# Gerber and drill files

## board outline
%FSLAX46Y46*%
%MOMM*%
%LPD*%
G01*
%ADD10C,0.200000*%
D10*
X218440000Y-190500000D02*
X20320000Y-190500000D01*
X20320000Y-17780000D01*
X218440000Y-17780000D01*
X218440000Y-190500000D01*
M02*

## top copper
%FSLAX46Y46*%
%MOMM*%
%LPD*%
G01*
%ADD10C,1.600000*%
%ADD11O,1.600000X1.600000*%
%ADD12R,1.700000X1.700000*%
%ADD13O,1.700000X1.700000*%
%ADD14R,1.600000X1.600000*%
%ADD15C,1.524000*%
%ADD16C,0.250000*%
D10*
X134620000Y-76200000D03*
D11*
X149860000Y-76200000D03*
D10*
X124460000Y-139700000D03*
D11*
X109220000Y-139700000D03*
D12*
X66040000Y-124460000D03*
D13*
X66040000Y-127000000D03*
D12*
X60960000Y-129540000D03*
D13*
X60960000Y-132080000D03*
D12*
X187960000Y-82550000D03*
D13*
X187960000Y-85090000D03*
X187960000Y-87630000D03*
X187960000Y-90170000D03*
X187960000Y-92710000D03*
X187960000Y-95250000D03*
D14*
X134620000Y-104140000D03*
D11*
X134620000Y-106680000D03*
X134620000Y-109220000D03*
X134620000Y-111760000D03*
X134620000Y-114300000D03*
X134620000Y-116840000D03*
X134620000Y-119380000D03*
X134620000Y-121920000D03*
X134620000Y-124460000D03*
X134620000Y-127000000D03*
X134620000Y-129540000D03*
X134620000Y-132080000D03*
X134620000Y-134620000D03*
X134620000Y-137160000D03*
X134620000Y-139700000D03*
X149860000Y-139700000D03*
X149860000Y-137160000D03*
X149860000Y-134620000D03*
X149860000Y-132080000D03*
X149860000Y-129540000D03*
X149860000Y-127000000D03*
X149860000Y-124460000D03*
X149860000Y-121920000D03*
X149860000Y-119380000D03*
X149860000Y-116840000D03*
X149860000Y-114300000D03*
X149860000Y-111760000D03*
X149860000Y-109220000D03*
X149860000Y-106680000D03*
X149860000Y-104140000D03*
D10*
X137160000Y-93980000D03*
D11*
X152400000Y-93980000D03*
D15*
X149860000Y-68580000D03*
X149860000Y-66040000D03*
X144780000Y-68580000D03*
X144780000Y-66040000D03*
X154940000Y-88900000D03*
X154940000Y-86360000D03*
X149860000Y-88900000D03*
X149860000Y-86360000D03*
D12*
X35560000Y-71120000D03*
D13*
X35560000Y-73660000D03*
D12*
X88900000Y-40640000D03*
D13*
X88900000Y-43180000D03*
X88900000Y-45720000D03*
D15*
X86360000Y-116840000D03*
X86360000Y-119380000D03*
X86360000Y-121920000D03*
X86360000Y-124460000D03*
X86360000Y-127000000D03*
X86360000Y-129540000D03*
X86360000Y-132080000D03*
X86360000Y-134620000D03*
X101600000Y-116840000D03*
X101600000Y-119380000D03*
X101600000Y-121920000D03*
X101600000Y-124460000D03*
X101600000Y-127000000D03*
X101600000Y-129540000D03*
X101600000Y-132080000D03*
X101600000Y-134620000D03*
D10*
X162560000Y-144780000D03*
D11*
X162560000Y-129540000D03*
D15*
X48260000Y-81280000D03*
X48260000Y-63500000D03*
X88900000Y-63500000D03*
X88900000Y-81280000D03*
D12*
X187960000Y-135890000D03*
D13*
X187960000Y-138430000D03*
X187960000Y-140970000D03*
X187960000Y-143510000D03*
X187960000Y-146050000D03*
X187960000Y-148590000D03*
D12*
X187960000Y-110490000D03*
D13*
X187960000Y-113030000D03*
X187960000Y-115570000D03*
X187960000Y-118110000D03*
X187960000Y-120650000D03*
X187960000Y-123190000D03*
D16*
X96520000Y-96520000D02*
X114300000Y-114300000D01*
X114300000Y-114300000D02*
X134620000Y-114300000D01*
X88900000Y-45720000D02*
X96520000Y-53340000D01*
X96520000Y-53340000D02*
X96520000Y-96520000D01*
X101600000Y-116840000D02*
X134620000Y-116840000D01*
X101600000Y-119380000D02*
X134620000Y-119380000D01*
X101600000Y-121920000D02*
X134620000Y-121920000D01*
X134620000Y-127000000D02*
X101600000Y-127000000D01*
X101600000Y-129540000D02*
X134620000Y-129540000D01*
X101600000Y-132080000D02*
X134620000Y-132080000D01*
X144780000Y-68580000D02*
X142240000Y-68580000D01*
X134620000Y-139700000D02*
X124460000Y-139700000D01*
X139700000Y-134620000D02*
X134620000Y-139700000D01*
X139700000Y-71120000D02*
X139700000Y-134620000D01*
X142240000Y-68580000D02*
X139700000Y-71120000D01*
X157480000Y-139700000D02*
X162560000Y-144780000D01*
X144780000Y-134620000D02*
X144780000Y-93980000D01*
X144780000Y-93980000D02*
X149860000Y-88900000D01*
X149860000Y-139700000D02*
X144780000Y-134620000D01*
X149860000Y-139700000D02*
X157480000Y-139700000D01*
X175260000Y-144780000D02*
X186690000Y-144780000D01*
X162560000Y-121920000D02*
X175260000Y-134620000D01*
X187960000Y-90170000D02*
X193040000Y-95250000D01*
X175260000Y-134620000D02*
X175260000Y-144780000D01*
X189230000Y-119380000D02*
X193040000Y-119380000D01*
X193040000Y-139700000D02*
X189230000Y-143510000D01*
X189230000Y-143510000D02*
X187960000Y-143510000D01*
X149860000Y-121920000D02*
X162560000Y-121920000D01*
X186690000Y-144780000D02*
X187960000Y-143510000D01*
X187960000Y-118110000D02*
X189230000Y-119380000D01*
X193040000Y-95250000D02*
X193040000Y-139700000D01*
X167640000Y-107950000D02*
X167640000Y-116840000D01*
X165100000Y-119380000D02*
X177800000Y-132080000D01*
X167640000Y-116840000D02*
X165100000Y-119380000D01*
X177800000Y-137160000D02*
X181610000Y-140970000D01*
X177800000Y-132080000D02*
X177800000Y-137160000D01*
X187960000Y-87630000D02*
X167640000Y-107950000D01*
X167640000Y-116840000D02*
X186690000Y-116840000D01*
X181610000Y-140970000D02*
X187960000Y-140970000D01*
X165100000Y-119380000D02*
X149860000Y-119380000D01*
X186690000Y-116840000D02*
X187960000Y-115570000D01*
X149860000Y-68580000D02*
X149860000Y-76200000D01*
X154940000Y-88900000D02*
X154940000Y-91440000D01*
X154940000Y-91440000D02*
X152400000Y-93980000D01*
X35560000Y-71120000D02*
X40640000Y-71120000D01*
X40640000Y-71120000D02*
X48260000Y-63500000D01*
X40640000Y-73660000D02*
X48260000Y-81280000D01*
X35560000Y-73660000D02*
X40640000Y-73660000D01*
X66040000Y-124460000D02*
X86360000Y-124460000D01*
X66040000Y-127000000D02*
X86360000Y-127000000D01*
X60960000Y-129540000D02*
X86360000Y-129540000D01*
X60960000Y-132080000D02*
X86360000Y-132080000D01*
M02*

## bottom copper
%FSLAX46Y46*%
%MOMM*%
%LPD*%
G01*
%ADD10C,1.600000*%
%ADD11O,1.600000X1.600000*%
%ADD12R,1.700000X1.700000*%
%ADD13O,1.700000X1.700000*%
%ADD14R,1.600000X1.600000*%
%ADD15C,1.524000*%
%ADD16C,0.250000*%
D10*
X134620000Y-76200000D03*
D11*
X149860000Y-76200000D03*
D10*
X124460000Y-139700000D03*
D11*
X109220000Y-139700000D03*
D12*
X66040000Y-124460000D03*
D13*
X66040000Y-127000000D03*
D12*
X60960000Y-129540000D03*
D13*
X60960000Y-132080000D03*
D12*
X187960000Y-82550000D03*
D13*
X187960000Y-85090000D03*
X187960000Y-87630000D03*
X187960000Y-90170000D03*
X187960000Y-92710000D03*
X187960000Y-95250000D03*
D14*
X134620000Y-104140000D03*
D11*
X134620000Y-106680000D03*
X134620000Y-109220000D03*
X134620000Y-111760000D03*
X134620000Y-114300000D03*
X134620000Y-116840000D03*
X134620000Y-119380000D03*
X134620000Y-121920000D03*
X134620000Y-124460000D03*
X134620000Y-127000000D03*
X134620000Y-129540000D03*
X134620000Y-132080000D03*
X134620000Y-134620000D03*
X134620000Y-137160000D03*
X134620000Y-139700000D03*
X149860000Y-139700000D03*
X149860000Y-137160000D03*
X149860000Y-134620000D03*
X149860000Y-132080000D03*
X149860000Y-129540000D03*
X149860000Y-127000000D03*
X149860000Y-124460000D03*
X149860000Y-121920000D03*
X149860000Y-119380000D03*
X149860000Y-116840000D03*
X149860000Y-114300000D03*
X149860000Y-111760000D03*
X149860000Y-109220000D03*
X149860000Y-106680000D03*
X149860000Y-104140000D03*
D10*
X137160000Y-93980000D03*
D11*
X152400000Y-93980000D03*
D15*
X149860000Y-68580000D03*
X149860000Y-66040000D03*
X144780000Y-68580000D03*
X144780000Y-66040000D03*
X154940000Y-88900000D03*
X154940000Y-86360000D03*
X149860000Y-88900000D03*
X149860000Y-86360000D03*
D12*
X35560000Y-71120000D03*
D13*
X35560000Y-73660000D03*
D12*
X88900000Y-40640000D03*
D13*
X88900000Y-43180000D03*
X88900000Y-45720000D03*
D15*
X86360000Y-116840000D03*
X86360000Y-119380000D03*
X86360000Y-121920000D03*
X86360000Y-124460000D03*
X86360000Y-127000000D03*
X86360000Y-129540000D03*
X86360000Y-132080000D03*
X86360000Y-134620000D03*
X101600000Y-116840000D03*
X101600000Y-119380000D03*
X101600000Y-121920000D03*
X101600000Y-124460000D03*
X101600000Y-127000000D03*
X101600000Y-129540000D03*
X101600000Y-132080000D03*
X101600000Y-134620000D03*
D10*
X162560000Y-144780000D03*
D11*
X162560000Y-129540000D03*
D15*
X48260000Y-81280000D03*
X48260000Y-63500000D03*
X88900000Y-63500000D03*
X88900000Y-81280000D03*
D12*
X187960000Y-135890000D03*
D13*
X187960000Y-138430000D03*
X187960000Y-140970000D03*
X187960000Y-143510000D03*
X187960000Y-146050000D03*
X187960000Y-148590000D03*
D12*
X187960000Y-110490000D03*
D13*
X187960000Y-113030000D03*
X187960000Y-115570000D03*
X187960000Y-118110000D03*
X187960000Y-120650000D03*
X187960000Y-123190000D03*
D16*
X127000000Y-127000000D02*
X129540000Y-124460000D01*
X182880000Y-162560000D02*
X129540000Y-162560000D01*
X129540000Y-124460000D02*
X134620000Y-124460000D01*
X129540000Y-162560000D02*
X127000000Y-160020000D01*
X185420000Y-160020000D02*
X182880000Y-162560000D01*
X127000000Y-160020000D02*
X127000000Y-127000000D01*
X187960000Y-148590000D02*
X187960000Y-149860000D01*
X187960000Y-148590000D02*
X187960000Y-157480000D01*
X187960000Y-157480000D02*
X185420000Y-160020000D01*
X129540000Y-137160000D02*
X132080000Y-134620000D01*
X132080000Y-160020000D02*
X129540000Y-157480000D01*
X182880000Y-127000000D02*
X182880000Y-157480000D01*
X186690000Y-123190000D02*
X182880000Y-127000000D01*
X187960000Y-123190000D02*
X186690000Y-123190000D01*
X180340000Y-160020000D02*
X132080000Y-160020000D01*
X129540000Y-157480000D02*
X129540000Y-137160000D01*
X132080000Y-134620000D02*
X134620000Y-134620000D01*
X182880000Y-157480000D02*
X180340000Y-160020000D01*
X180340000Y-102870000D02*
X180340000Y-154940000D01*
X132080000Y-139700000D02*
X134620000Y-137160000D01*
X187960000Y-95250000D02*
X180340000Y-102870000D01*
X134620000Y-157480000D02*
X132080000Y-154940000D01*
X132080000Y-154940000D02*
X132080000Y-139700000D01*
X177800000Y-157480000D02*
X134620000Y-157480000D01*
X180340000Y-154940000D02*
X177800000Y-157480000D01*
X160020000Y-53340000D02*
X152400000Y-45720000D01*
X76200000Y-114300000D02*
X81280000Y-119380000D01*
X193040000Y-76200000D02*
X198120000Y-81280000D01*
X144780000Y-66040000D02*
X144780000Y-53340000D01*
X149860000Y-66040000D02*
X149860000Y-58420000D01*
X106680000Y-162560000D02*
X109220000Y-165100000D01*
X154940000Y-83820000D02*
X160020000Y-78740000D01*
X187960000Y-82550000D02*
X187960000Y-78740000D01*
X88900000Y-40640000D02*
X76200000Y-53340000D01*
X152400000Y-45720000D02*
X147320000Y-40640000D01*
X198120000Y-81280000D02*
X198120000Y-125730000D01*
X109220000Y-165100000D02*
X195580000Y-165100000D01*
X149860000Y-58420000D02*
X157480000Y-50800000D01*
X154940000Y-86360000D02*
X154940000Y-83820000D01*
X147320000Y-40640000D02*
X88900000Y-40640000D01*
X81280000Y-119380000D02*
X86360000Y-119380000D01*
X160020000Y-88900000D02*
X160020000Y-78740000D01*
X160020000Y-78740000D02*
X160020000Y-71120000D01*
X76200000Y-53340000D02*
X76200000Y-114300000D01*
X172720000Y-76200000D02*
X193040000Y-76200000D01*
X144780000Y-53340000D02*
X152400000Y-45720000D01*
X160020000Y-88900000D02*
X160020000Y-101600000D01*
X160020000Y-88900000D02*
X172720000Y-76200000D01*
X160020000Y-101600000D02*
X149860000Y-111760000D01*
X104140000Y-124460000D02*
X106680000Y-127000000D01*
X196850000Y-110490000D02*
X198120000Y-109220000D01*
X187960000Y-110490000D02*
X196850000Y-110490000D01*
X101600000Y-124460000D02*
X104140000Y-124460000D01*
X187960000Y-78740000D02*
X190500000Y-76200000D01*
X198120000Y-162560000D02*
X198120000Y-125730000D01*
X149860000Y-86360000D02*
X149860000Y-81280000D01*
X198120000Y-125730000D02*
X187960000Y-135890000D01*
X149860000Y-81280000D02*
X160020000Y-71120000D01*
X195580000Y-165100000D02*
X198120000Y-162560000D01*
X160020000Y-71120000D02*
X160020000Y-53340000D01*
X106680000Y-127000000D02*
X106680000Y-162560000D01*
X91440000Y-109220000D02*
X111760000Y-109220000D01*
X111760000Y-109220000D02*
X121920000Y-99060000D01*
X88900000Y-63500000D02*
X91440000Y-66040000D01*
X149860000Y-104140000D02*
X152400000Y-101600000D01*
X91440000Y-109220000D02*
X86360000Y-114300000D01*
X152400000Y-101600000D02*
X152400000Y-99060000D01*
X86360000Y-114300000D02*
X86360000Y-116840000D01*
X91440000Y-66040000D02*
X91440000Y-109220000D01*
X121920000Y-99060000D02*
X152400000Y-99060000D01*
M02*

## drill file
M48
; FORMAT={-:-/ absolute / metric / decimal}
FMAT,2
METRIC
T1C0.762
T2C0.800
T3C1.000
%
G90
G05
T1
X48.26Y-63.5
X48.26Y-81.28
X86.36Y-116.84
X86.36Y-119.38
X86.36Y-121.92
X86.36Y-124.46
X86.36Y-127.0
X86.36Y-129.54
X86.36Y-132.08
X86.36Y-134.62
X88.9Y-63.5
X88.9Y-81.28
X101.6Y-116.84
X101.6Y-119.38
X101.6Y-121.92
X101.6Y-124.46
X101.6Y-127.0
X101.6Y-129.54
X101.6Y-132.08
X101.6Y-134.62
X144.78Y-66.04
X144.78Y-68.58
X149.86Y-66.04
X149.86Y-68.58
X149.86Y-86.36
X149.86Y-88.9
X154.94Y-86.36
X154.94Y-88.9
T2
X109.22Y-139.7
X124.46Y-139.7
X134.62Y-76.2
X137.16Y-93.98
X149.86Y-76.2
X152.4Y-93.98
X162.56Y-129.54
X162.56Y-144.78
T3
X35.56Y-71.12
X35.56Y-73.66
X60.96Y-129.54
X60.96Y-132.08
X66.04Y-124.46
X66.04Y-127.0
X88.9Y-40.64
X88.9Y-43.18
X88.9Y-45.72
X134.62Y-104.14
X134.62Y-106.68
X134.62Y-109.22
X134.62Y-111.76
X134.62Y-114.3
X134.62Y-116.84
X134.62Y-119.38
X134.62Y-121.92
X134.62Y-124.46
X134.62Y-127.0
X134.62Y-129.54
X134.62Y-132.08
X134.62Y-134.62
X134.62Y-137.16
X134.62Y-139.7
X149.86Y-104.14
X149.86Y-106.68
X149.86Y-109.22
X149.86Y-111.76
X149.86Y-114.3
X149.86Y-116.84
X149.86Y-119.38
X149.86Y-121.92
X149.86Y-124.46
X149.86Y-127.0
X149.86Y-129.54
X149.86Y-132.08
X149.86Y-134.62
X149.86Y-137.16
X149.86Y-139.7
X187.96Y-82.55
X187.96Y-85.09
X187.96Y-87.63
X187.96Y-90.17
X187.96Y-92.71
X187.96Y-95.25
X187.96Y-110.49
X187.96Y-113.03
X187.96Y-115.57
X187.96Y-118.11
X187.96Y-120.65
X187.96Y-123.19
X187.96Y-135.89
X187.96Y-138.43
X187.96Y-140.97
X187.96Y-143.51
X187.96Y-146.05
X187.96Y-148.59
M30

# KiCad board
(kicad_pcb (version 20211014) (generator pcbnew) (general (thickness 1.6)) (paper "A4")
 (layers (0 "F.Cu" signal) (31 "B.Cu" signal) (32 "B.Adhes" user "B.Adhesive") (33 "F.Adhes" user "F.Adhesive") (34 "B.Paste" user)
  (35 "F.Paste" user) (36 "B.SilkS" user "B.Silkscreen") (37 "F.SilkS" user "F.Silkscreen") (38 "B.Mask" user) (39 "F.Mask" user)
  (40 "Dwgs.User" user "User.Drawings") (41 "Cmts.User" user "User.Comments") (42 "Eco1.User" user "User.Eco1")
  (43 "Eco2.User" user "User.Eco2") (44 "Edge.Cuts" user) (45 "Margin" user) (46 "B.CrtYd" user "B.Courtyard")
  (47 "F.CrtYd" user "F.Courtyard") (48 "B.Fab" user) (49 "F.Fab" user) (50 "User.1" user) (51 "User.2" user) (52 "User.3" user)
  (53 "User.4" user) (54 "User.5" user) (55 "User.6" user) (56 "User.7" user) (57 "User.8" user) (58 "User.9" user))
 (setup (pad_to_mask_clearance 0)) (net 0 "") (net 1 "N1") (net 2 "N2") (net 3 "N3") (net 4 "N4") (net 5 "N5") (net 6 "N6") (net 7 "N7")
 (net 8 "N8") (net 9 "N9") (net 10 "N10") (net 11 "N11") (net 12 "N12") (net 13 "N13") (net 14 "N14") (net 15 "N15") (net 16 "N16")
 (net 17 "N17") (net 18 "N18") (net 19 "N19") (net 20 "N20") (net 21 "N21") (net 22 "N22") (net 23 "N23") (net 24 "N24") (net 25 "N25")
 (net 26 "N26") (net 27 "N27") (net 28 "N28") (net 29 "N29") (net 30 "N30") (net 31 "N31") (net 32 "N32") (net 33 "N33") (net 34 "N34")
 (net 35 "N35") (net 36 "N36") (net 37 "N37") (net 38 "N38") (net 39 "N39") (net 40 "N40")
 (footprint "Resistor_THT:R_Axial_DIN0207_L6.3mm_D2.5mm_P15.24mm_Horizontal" (layer "F.Cu") (at 134.62 76.2)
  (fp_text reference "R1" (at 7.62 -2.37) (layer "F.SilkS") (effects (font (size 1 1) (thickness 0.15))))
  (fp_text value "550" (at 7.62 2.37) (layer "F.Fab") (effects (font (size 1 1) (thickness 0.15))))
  (pad "1" thru_hole circle (at 0 0) (size 1.6 1.6) (drill 0.8) (layers *.Cu *.Mask) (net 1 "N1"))
  (pad "2" thru_hole oval (at 15.24 0) (size 1.6 1.6) (drill 0.8) (layers *.Cu *.Mask) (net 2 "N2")))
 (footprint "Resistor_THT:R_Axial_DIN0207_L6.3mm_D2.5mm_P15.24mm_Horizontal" (layer "F.Cu") (at 124.46 139.7 180)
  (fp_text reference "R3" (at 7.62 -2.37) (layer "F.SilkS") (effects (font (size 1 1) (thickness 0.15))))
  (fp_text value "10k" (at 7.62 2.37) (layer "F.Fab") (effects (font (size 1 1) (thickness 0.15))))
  (pad "1" thru_hole circle (at 0 0 180) (size 1.6 1.6) (drill 0.8) (layers *.Cu *.Mask) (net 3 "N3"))
  (pad "2" thru_hole oval (at 15.24 0 180) (size 1.6 1.6) (drill 0.8) (layers *.Cu *.Mask) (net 1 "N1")))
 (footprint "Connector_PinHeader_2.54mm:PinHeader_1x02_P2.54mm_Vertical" (layer "F.Cu") (at 66.04 124.46)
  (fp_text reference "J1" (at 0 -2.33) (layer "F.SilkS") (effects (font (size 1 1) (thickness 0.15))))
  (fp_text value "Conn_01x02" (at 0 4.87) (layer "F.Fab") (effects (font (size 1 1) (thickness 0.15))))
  (pad "1" thru_hole rect (at 0 0) (size 1.7 1.7) (drill 1) (layers *.Cu *.Mask) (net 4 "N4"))
  (pad "2" thru_hole oval (at 0 2.54) (size 1.7 1.7) (drill 1) (layers *.Cu *.Mask) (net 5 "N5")))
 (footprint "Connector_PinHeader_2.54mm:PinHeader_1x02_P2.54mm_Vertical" (layer "F.Cu") (at 60.96 129.54)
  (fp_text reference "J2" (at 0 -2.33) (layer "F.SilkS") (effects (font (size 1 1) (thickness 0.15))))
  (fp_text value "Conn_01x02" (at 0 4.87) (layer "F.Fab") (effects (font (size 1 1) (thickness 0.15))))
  (pad "1" thru_hole rect (at 0 0) (size 1.7 1.7) (drill 1) (layers *.Cu *.Mask) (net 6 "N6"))
  (pad "2" thru_hole oval (at 0 2.54) (size 1.7 1.7) (drill 1) (layers *.Cu *.Mask) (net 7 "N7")))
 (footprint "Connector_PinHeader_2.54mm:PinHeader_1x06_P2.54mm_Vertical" (layer "F.Cu") (at 187.96 82.55)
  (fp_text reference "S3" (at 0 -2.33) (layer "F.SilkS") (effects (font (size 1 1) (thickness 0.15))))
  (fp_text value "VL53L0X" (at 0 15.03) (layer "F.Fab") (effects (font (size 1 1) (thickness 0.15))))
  (pad "1" thru_hole rect (at 0 0) (size 1.7 1.7) (drill 1) (layers *.Cu *.Mask) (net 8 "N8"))
  (pad "2" thru_hole oval (at 0 2.54) (size 1.7 1.7) (drill 1) (layers *.Cu *.Mask) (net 1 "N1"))
  (pad "3" thru_hole oval (at 0 5.08) (size 1.7 1.7) (drill 1) (layers *.Cu *.Mask) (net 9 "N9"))
  (pad "4" thru_hole oval (at 0 7.62) (size 1.7 1.7) (drill 1) (layers *.Cu *.Mask) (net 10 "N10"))
  (pad "5" thru_hole oval (at 0 10.16) (size 1.7 1.7) (drill 1) (layers *.Cu *.Mask) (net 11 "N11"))
  (pad "6" thru_hole oval (at 0 12.7) (size 1.7 1.7) (drill 1) (layers *.Cu *.Mask) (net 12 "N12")))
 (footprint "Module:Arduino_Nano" (layer "F.Cu") (at 134.62 104.14)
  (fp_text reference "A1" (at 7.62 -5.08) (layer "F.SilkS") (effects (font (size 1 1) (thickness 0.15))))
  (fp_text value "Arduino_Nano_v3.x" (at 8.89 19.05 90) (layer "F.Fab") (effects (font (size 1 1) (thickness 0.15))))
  (pad "1" thru_hole rect (at 0 0) (size 1.6 1.6) (drill 1) (layers *.Cu *.Mask) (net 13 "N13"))
  (pad "2" thru_hole oval (at 0 2.54) (size 1.6 1.6) (drill 1) (layers *.Cu *.Mask) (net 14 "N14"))
  (pad "3" thru_hole oval (at 0 5.08) (size 1.6 1.6) (drill 1) (layers *.Cu *.Mask) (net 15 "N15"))
  (pad "4" thru_hole oval (at 0 7.62) (size 1.6 1.6) (drill 1) (layers *.Cu *.Mask) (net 1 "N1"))
  (pad "5" thru_hole oval (at 0 10.16) (size 1.6 1.6) (drill 1) (layers *.Cu *.Mask) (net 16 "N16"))
  (pad "6" thru_hole oval (at 0 12.7) (size 1.6 1.6) (drill 1) (layers *.Cu *.Mask) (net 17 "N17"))
  (pad "7" thru_hole oval (at 0 15.24) (size 1.6 1.6) (drill 1) (layers *.Cu *.Mask) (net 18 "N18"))
  (pad "8" thru_hole oval (at 0 17.78) (size 1.6 1.6) (drill 1) (layers *.Cu *.Mask) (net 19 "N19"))
  (pad "9" thru_hole oval (at 0 20.32) (size 1.6 1.6) (drill 1) (layers *.Cu *.Mask) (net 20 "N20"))
  (pad "10" thru_hole oval (at 0 22.86) (size 1.6 1.6) (drill 1) (layers *.Cu *.Mask) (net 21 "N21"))
  (pad "11" thru_hole oval (at 0 25.4) (size 1.6 1.6) (drill 1) (layers *.Cu *.Mask) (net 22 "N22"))
  (pad "12" thru_hole oval (at 0 27.94) (size 1.6 1.6) (drill 1) (layers *.Cu *.Mask) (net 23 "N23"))
  (pad "13" thru_hole oval (at 0 30.48) (size 1.6 1.6) (drill 1) (layers *.Cu *.Mask) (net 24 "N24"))
  (pad "14" thru_hole oval (at 0 33.02) (size 1.6 1.6) (drill 1) (layers *.Cu *.Mask) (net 12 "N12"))
  (pad "15" thru_hole oval (at 0 35.56) (size 1.6 1.6) (drill 1) (layers *.Cu *.Mask) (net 3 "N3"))
  (pad "16" thru_hole oval (at 15.24 35.56) (size 1.6 1.6) (drill 1) (layers *.Cu *.Mask) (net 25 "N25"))
  (pad "17" thru_hole oval (at 15.24 33.02) (size 1.6 1.6) (drill 1) (layers *.Cu *.Mask) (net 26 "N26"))
  (pad "18" thru_hole oval (at 15.24 30.48) (size 1.6 1.6) (drill 1) (layers *.Cu *.Mask) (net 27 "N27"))
  (pad "19" thru_hole oval (at 15.24 27.94) (size 1.6 1.6) (drill 1) (layers *.Cu *.Mask) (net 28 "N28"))
  (pad "20" thru_hole oval (at 15.24 25.4) (size 1.6 1.6) (drill 1) (layers *.Cu *.Mask) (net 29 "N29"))
  (pad "21" thru_hole oval (at 15.24 22.86) (size 1.6 1.6) (drill 1) (layers *.Cu *.Mask) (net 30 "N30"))
  (pad "22" thru_hole oval (at 15.24 20.32) (size 1.6 1.6) (drill 1) (layers *.Cu *.Mask) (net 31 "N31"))
  (pad "23" thru_hole oval (at 15.24 17.78) (size 1.6 1.6) (drill 1) (layers *.Cu *.Mask) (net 10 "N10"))
  (pad "24" thru_hole oval (at 15.24 15.24) (size 1.6 1.6) (drill 1) (layers *.Cu *.Mask) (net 9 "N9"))
  (pad "25" thru_hole oval (at 15.24 12.7) (size 1.6 1.6) (drill 1) (layers *.Cu *.Mask) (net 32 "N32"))
  (pad "26" thru_hole oval (at 15.24 10.16) (size 1.6 1.6) (drill 1) (layers *.Cu *.Mask) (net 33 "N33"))
  (pad "27" thru_hole oval (at 15.24 7.62) (size 1.6 1.6) (drill 1) (layers *.Cu *.Mask) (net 8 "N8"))
  (pad "28" thru_hole oval (at 15.24 5.08) (size 1.6 1.6) (drill 1) (layers *.Cu *.Mask) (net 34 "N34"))
  (pad "29" thru_hole oval (at 15.24 2.54) (size 1.6 1.6) (drill 1) (layers *.Cu *.Mask) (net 1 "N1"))
  (pad "30" thru_hole oval (at 15.24 0) (size 1.6 1.6) (drill 1) (layers *.Cu *.Mask) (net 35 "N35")))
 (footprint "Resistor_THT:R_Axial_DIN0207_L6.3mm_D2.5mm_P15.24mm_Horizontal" (layer "F.Cu") (at 137.16 93.98)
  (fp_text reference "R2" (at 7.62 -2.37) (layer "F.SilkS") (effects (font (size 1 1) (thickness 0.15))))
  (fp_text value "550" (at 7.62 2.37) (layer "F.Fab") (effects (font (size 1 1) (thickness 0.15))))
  (pad "1" thru_hole circle (at 0 0) (size 1.6 1.6) (drill 0.8) (layers *.Cu *.Mask) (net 1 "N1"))
  (pad "2" thru_hole oval (at 15.24 0) (size 1.6 1.6) (drill 0.8) (layers *.Cu *.Mask) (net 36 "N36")))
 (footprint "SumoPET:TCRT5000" (layer "F.Cu") (at 147.32 68.58)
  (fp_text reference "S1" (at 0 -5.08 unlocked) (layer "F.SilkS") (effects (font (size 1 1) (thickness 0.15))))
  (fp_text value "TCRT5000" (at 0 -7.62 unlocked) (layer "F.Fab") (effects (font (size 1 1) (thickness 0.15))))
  (pad "1" thru_hole circle (at 2.54 0) (size 1.524 1.524) (drill 0.762) (layers *.Cu *.Mask) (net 2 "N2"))
  (pad "2" thru_hole circle (at 2.54 -2.54) (size 1.524 1.524) (drill 0.762) (layers *.Cu *.Mask) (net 8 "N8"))
  (pad "3" thru_hole circle (at -2.54 0) (size 1.524 1.524) (drill 0.762) (layers *.Cu *.Mask) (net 3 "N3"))
  (pad "4" thru_hole circle (at -2.54 -2.54) (size 1.524 1.524) (drill 0.762) (layers *.Cu *.Mask) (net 8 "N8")))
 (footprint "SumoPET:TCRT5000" (layer "F.Cu") (at 152.4 88.9)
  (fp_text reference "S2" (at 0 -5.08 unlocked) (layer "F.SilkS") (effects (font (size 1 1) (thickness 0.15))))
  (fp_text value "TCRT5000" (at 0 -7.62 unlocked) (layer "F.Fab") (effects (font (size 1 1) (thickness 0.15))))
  (pad "1" thru_hole circle (at 2.54 0) (size 1.524 1.524) (drill 0.762) (layers *.Cu *.Mask) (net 36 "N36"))
  (pad "2" thru_hole circle (at 2.54 -2.54) (size 1.524 1.524) (drill 0.762) (layers *.Cu *.Mask) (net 8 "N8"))
  (pad "3" thru_hole circle (at -2.54 0) (size 1.524 1.524) (drill 0.762) (layers *.Cu *.Mask) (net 25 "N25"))
  (pad "4" thru_hole circle (at -2.54 -2.54) (size 1.524 1.524) (drill 0.762) (layers *.Cu *.Mask) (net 8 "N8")))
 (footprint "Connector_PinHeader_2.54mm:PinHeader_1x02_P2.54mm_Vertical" (layer "F.Cu") (at 35.56 71.12)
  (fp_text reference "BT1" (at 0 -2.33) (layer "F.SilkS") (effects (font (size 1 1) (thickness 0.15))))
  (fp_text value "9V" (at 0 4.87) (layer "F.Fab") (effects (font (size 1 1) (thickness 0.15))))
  (pad "1" thru_hole rect (at 0 0) (size 1.7 1.7) (drill 1) (layers *.Cu *.Mask) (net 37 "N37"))
  (pad "2" thru_hole oval (at 0 2.54) (size 1.7 1.7) (drill 1) (layers *.Cu *.Mask) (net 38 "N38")))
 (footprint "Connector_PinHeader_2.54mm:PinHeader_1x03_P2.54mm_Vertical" (layer "F.Cu") (at 88.9 40.64)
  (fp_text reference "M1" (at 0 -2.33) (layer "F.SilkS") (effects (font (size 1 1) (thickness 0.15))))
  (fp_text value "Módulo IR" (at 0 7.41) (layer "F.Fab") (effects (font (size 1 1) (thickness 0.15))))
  (pad "1" thru_hole rect (at 0 0) (size 1.7 1.7) (drill 1) (layers *.Cu *.Mask) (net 8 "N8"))
  (pad "2" thru_hole oval (at 0 2.54) (size 1.7 1.7) (drill 1) (layers *.Cu *.Mask) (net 1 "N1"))
  (pad "3" thru_hole oval (at 0 5.08) (size 1.7 1.7) (drill 1) (layers *.Cu *.Mask) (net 16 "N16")))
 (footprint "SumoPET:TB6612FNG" (layer "F.Cu") (at 93.98 127)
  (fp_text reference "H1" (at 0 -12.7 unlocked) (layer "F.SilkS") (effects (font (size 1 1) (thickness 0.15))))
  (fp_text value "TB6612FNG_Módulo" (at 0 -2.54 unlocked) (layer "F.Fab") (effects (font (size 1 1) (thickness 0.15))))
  (pad "1" thru_hole circle (at -7.62 -10.16) (size 1.524 1.524) (drill 0.762) (layers *.Cu *.Mask) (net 35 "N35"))
  (pad "2" thru_hole circle (at -7.62 -7.62) (size 1.524 1.524) (drill 0.762) (layers *.Cu *.Mask) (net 8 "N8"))
  (pad "3" thru_hole circle (at -7.62 -5.08) (size 1.524 1.524) (drill 0.762) (layers *.Cu *.Mask) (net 1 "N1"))
  (pad "4" thru_hole circle (at -7.62 -2.54) (size 1.524 1.524) (drill 0.762) (layers *.Cu *.Mask) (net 4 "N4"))
  (pad "5" thru_hole circle (at -7.62 0) (size 1.524 1.524) (drill 0.762) (layers *.Cu *.Mask) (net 5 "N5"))
  (pad "6" thru_hole circle (at -7.62 2.54) (size 1.524 1.524) (drill 0.762) (layers *.Cu *.Mask) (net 6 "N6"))
  (pad "7" thru_hole circle (at -7.62 5.08) (size 1.524 1.524) (drill 0.762) (layers *.Cu *.Mask) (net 7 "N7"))
  (pad "8" thru_hole circle (at -7.62 7.62) (size 1.524 1.524) (drill 0.762) (layers *.Cu *.Mask) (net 1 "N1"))
  (pad "9" thru_hole circle (at 7.62 -10.16) (size 1.524 1.524) (drill 0.762) (layers *.Cu *.Mask) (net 17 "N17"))
  (pad "10" thru_hole circle (at 7.62 -7.62) (size 1.524 1.524) (drill 0.762) (layers *.Cu *.Mask) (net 18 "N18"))
  (pad "11" thru_hole circle (at 7.62 -5.08) (size 1.524 1.524) (drill 0.762) (layers *.Cu *.Mask) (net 19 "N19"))
  (pad "12" thru_hole circle (at 7.62 -2.54) (size 1.524 1.524) (drill 0.762) (layers *.Cu *.Mask) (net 8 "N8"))
  (pad "13" thru_hole circle (at 7.62 0) (size 1.524 1.524) (drill 0.762) (layers *.Cu *.Mask) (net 21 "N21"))
  (pad "14" thru_hole circle (at 7.62 2.54) (size 1.524 1.524) (drill 0.762) (layers *.Cu *.Mask) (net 22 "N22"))
  (pad "15" thru_hole circle (at 7.62 5.08) (size 1.524 1.524) (drill 0.762) (layers *.Cu *.Mask) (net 23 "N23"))
  (pad "16" thru_hole circle (at 7.62 7.62) (size 1.524 1.524) (drill 0.762) (layers *.Cu *.Mask) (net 1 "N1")))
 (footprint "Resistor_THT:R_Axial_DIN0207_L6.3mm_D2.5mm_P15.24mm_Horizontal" (layer "F.Cu") (at 162.56 144.78 90)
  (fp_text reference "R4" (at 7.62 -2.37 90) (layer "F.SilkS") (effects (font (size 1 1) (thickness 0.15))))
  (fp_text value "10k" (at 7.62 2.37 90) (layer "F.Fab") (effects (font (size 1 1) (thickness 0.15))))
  (pad "1" thru_hole circle (at 0 0 90) (size 1.6 1.6) (drill 0.8) (layers *.Cu *.Mask) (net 25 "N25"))
  (pad "2" thru_hole oval (at 15.24 0 90) (size 1.6 1.6) (drill 0.8) (layers *.Cu *.Mask) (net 1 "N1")))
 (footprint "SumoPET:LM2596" (layer "F.Cu") (at 68.58 73.66)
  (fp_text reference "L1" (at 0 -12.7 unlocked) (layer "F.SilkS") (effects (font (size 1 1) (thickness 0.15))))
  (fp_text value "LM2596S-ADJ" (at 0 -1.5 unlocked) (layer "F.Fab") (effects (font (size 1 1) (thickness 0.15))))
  (pad "1" thru_hole circle (at -20.32 7.62) (size 1.524 1.524) (drill 0.762) (layers *.Cu *.Mask) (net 38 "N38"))
  (pad "2" thru_hole circle (at -20.32 -10.16) (size 1.524 1.524) (drill 0.762) (layers *.Cu *.Mask) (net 37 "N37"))
  (pad "3" thru_hole circle (at 20.32 -10.16) (size 1.524 1.524) (drill 0.762) (layers *.Cu *.Mask) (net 35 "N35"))
  (pad "4" thru_hole circle (at 20.32 7.62) (size 1.524 1.524) (drill 0.762) (layers *.Cu *.Mask) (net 1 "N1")))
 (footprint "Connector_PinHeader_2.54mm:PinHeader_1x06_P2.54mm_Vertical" (layer "F.Cu") (at 187.96 135.89)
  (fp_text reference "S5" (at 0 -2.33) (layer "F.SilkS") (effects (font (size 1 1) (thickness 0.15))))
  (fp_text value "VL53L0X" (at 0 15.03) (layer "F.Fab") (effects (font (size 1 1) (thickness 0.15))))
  (pad "1" thru_hole rect (at 0 0) (size 1.7 1.7) (drill 1) (layers *.Cu *.Mask) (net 8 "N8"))
  (pad "2" thru_hole oval (at 0 2.54) (size 1.7 1.7) (drill 1) (layers *.Cu *.Mask) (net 1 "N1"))
  (pad "3" thru_hole oval (at 0 5.08) (size 1.7 1.7) (drill 1) (layers *.Cu *.Mask) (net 9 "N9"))
  (pad "4" thru_hole oval (at 0 7.62) (size 1.7 1.7) (drill 1) (layers *.Cu *.Mask) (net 10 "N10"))
  (pad "5" thru_hole oval (at 0 10.16) (size 1.7 1.7) (drill 1) (layers *.Cu *.Mask) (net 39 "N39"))
  (pad "6" thru_hole oval (at 0 12.7) (size 1.7 1.7) (drill 1) (layers *.Cu *.Mask) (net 20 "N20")))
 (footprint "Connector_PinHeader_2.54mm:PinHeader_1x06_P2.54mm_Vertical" (layer "F.Cu") (at 187.96 110.49)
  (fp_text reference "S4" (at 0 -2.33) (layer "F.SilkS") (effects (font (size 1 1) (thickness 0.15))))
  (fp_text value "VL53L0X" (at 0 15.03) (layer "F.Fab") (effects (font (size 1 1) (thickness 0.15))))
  (pad "1" thru_hole rect (at 0 0) (size 1.7 1.7) (drill 1) (layers *.Cu *.Mask) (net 8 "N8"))
  (pad "2" thru_hole oval (at 0 2.54) (size 1.7 1.7) (drill 1) (layers *.Cu *.Mask) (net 1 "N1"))
  (pad "3" thru_hole oval (at 0 5.08) (size 1.7 1.7) (drill 1) (layers *.Cu *.Mask) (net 9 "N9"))
  (pad "4" thru_hole oval (at 0 7.62) (size 1.7 1.7) (drill 1) (layers *.Cu *.Mask) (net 10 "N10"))
  (pad "5" thru_hole oval (at 0 10.16) (size 1.7 1.7) (drill 1) (layers *.Cu *.Mask) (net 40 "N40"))
  (pad "6" thru_hole oval (at 0 12.7) (size 1.7 1.7) (drill 1) (layers *.Cu *.Mask) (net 24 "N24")))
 (gr_poly (pts (xy 218.44 190.5) (xy 20.32 190.5) (xy 20.32 17.78) (xy 218.44 17.78)) (layer "Edge.Cuts") (width 0.2) (fill none))
 (segment (start 96.52 96.52) (end 114.3 114.3) (width 0.25) (layer "F.Cu") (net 16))
 (segment (start 114.3 114.3) (end 134.62 114.3) (width 0.25) (layer "F.Cu") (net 16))
 (segment (start 88.9 45.72) (end 96.52 53.34) (width 0.25) (layer "F.Cu") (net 16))
 (segment (start 96.52 53.34) (end 96.52 96.52) (width 0.25) (layer "F.Cu") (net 16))
 (segment (start 101.6 116.84) (end 134.62 116.84) (width 0.25) (layer "F.Cu") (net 17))
 (segment (start 101.6 119.38) (end 134.62 119.38) (width 0.25) (layer "F.Cu") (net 18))
 (segment (start 101.6 121.92) (end 134.62 121.92) (width 0.25) (layer "F.Cu") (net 19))
 (segment (start 127 127) (end 129.54 124.46) (width 0.25) (layer "B.Cu") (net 20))
 (segment (start 182.88 162.56) (end 129.54 162.56) (width 0.25) (layer "B.Cu") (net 20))
 (segment (start 129.54 124.46) (end 134.62 124.46) (width 0.25) (layer "B.Cu") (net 20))
 (segment (start 129.54 162.56) (end 127 160.02) (width 0.25) (layer "B.Cu") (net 20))
 (segment (start 185.42 160.02) (end 182.88 162.56) (width 0.25) (layer "B.Cu") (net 20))
 (segment (start 127 160.02) (end 127 127) (width 0.25) (layer "B.Cu") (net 20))
 (segment (start 187.96 148.59) (end 187.96 149.86) (width 0.25) (layer "B.Cu") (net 20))
 (segment (start 187.96 148.59) (end 187.96 157.48) (width 0.25) (layer "B.Cu") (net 20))
 (segment (start 187.96 157.48) (end 185.42 160.02) (width 0.25) (layer "B.Cu") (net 20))
 (segment (start 134.62 127) (end 101.6 127) (width 0.25) (layer "F.Cu") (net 21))
 (segment (start 101.6 129.54) (end 134.62 129.54) (width 0.25) (layer "F.Cu") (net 22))
 (segment (start 101.6 132.08) (end 134.62 132.08) (width 0.25) (layer "F.Cu") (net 23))
 (segment (start 129.54 137.16) (end 132.08 134.62) (width 0.25) (layer "B.Cu") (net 24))
 (segment (start 132.08 160.02) (end 129.54 157.48) (width 0.25) (layer "B.Cu") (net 24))
 (segment (start 182.88 127) (end 182.88 157.48) (width 0.25) (layer "B.Cu") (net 24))
 (segment (start 186.69 123.19) (end 182.88 127) (width 0.25) (layer "B.Cu") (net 24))
 (segment (start 187.96 123.19) (end 186.69 123.19) (width 0.25) (layer "B.Cu") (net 24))
 (segment (start 180.34 160.02) (end 132.08 160.02) (width 0.25) (layer "B.Cu") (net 24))
 (segment (start 129.54 157.48) (end 129.54 137.16) (width 0.25) (layer "B.Cu") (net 24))
 (segment (start 132.08 134.62) (end 134.62 134.62) (width 0.25) (layer "B.Cu") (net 24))
 (segment (start 182.88 157.48) (end 180.34 160.02) (width 0.25) (layer "B.Cu") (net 24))
 (segment (start 180.34 102.87) (end 180.34 154.94) (width 0.25) (layer "B.Cu") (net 12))
 (segment (start 132.08 139.7) (end 134.62 137.16) (width 0.25) (layer "B.Cu") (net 12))
 (segment (start 187.96 95.25) (end 180.34 102.87) (width 0.25) (layer "B.Cu") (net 12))
 (segment (start 134.62 157.48) (end 132.08 154.94) (width 0.25) (layer "B.Cu") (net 12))
 (segment (start 132.08 154.94) (end 132.08 139.7) (width 0.25) (layer "B.Cu") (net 12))
 (segment (start 177.8 157.48) (end 134.62 157.48) (width 0.25) (layer "B.Cu") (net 12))
 (segment (start 180.34 154.94) (end 177.8 157.48) (width 0.25) (layer "B.Cu") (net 12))
 (segment (start 144.78 68.58) (end 142.24 68.58) (width 0.25) (layer "F.Cu") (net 3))
 (segment (start 134.62 139.7) (end 124.46 139.7) (width 0.25) (layer "F.Cu") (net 3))
 (segment (start 139.7 134.62) (end 134.62 139.7) (width 0.25) (layer "F.Cu") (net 3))
 (segment (start 139.7 71.12) (end 139.7 134.62) (width 0.25) (layer "F.Cu") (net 3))
 (segment (start 142.24 68.58) (end 139.7 71.12) (width 0.25) (layer "F.Cu") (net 3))
 (segment (start 157.48 139.7) (end 162.56 144.78) (width 0.25) (layer "F.Cu") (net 25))
 (segment (start 144.78 134.62) (end 144.78 93.98) (width 0.25) (layer "F.Cu") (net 25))
 (segment (start 144.78 93.98) (end 149.86 88.9) (width 0.25) (layer "F.Cu") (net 25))
 (segment (start 149.86 139.7) (end 144.78 134.62) (width 0.25) (layer "F.Cu") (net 25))
 (segment (start 149.86 139.7) (end 157.48 139.7) (width 0.25) (layer "F.Cu") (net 25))
 (segment (start 175.26 144.78) (end 186.69 144.78) (width 0.25) (layer "F.Cu") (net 10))
 (segment (start 162.56 121.92) (end 175.26 134.62) (width 0.25) (layer "F.Cu") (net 10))
 (segment (start 187.96 90.17) (end 193.04 95.25) (width 0.25) (layer "F.Cu") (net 10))
 (segment (start 175.26 134.62) (end 175.26 144.78) (width 0.25) (layer "F.Cu") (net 10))
 (segment (start 189.23 119.38) (end 193.04 119.38) (width 0.25) (layer "F.Cu") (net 10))
 (segment (start 193.04 139.7) (end 189.23 143.51) (width 0.25) (layer "F.Cu") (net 10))
 (segment (start 189.23 143.51) (end 187.96 143.51) (width 0.25) (layer "F.Cu") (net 10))
 (segment (start 149.86 121.92) (end 162.56 121.92) (width 0.25) (layer "F.Cu") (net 10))
 (segment (start 186.69 144.78) (end 187.96 143.51) (width 0.25) (layer "F.Cu") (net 10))
 (segment (start 187.96 118.11) (end 189.23 119.38) (width 0.25) (layer "F.Cu") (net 10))
 (segment (start 193.04 95.25) (end 193.04 139.7) (width 0.25) (layer "F.Cu") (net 10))
 (segment (start 167.64 107.95) (end 167.64 116.84) (width 0.25) (layer "F.Cu") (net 9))
 (segment (start 165.1 119.38) (end 177.8 132.08) (width 0.25) (layer "F.Cu") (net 9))
 (segment (start 167.64 116.84) (end 165.1 119.38) (width 0.25) (layer "F.Cu") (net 9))
 (segment (start 177.8 137.16) (end 181.61 140.97) (width 0.25) (layer "F.Cu") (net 9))
 (segment (start 177.8 132.08) (end 177.8 137.16) (width 0.25) (layer "F.Cu") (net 9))
 (segment (start 187.96 87.63) (end 167.64 107.95) (width 0.25) (layer "F.Cu") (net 9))
 (segment (start 167.64 116.84) (end 186.69 116.84) (width 0.25) (layer "F.Cu") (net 9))
 (segment (start 181.61 140.97) (end 187.96 140.97) (width 0.25) (layer "F.Cu") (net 9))
 (segment (start 165.1 119.38) (end 149.86 119.38) (width 0.25) (layer "F.Cu") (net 9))
 (segment (start 186.69 116.84) (end 187.96 115.57) (width 0.25) (layer "F.Cu") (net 9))
 (segment (start 160.02 53.34) (end 152.4 45.72) (width 0.25) (layer "B.Cu") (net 8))
 (segment (start 76.2 114.3) (end 81.28 119.38) (width 0.25) (layer "B.Cu") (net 8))
 (segment (start 193.04 76.2) (end 198.12 81.28) (width 0.25) (layer "B.Cu") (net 8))
 (segment (start 144.78 66.04) (end 144.78 53.34) (width 0.25) (layer "B.Cu") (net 8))
 (segment (start 149.86 66.04) (end 149.86 58.42) (width 0.25) (layer "B.Cu") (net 8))
 (segment (start 106.68 162.56) (end 109.22 165.1) (width 0.25) (layer "B.Cu") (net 8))
 (segment (start 154.94 83.82) (end 160.02 78.74) (width 0.25) (layer "B.Cu") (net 8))
 (segment (start 187.96 82.55) (end 187.96 78.74) (width 0.25) (layer "B.Cu") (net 8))
 (segment (start 88.9 40.64) (end 76.2 53.34) (width 0.25) (layer "B.Cu") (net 8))
 (segment (start 152.4 45.72) (end 147.32 40.64) (width 0.25) (layer "B.Cu") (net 8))
 (segment (start 198.12 81.28) (end 198.12 125.73) (width 0.25) (layer "B.Cu") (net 8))
 (segment (start 109.22 165.1) (end 195.58 165.1) (width 0.25) (layer "B.Cu") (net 8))
 (segment (start 149.86 58.42) (end 157.48 50.8) (width 0.25) (layer "B.Cu") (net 8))
 (segment (start 154.94 86.36) (end 154.94 83.82) (width 0.25) (layer "B.Cu") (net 8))
 (segment (start 147.32 40.64) (end 88.9 40.64) (width 0.25) (layer "B.Cu") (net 8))
 (segment (start 81.28 119.38) (end 86.36 119.38) (width 0.25) (layer "B.Cu") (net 8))
 (segment (start 160.02 88.9) (end 160.02 78.74) (width 0.25) (layer "B.Cu") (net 8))
 (segment (start 160.02 78.74) (end 160.02 71.12) (width 0.25) (layer "B.Cu") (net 8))
 (segment (start 76.2 53.34) (end 76.2 114.3) (width 0.25) (layer "B.Cu") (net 8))
 (segment (start 172.72 76.2) (end 193.04 76.2) (width 0.25) (layer "B.Cu") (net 8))
 (segment (start 144.78 53.34) (end 152.4 45.72) (width 0.25) (layer "B.Cu") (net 8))
 (segment (start 160.02 88.9) (end 160.02 101.6) (width 0.25) (layer "B.Cu") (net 8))
 (segment (start 160.02 88.9) (end 172.72 76.2) (width 0.25) (layer "B.Cu") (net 8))
 (segment (start 160.02 101.6) (end 149.86 111.76) (width 0.25) (layer "B.Cu") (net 8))
 (segment (start 104.14 124.46) (end 106.68 127) (width 0.25) (layer "B.Cu") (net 8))
 (segment (start 196.85 110.49) (end 198.12 109.22) (width 0.25) (layer "B.Cu") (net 8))
 (segment (start 187.96 110.49) (end 196.85 110.49) (width 0.25) (layer "B.Cu") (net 8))
 (segment (start 101.6 124.46) (end 104.14 124.46) (width 0.25) (layer "B.Cu") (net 8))
 (segment (start 187.96 78.74) (end 190.5 76.2) (width 0.25) (layer "B.Cu") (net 8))
 (segment (start 198.12 162.56) (end 198.12 125.73) (width 0.25) (layer "B.Cu") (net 8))
 (segment (start 149.86 86.36) (end 149.86 81.28) (width 0.25) (layer "B.Cu") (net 8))
 (segment (start 198.12 125.73) (end 187.96 135.89) (width 0.25) (layer "B.Cu") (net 8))
 (segment (start 149.86 81.28) (end 160.02 71.12) (width 0.25) (layer "B.Cu") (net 8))
 (segment (start 195.58 165.1) (end 198.12 162.56) (width 0.25) (layer "B.Cu") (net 8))
 (segment (start 160.02 71.12) (end 160.02 53.34) (width 0.25) (layer "B.Cu") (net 8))
 (segment (start 106.68 127) (end 106.68 162.56) (width 0.25) (layer "B.Cu") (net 8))
 (segment (start 91.44 109.22) (end 111.76 109.22) (width 0.25) (layer "B.Cu") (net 35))
 (segment (start 111.76 109.22) (end 121.92 99.06) (width 0.25) (layer "B.Cu") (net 35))
 (segment (start 88.9 63.5) (end 91.44 66.04) (width 0.25) (layer "B.Cu") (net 35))
 (segment (start 149.86 104.14) (end 152.4 101.6) (width 0.25) (layer "B.Cu") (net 35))
 (segment (start 91.44 109.22) (end 86.36 114.3) (width 0.25) (layer "B.Cu") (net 35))
 (segment (start 152.4 101.6) (end 152.4 99.06) (width 0.25) (layer "B.Cu") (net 35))
 (segment (start 86.36 114.3) (end 86.36 116.84) (width 0.25) (layer "B.Cu") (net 35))
 (segment (start 91.44 66.04) (end 91.44 109.22) (width 0.25) (layer "B.Cu") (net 35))
 (segment (start 121.92 99.06) (end 152.4 99.06) (width 0.25) (layer "B.Cu") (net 35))
 (segment (start 149.86 68.58) (end 149.86 76.2) (width 0.25) (layer "F.Cu") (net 2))
 (segment (start 154.94 88.9) (end 154.94 91.44) (width 0.25) (layer "F.Cu") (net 36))
 (segment (start 154.94 91.44) (end 152.4 93.98) (width 0.25) (layer "F.Cu") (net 36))
 (segment (start 35.56 71.12) (end 40.64 71.12) (width 0.25) (layer "F.Cu") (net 37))
 (segment (start 40.64 71.12) (end 48.26 63.5) (width 0.25) (layer "F.Cu") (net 37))
 (segment (start 40.64 73.66) (end 48.26 81.28) (width 0.25) (layer "F.Cu") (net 38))
 (segment (start 35.56 73.66) (end 40.64 73.66) (width 0.25) (layer "F.Cu") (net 38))
 (segment (start 66.04 124.46) (end 86.36 124.46) (width 0.25) (layer "F.Cu") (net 4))
 (segment (start 66.04 127) (end 86.36 127) (width 0.25) (layer "F.Cu") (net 5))
 (segment (start 60.96 129.54) (end 86.36 129.54) (width 0.25) (layer "F.Cu") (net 6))
 (segment (start 60.96 132.08) (end 86.36 132.08) (width 0.25) (layer "F.Cu") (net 7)))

